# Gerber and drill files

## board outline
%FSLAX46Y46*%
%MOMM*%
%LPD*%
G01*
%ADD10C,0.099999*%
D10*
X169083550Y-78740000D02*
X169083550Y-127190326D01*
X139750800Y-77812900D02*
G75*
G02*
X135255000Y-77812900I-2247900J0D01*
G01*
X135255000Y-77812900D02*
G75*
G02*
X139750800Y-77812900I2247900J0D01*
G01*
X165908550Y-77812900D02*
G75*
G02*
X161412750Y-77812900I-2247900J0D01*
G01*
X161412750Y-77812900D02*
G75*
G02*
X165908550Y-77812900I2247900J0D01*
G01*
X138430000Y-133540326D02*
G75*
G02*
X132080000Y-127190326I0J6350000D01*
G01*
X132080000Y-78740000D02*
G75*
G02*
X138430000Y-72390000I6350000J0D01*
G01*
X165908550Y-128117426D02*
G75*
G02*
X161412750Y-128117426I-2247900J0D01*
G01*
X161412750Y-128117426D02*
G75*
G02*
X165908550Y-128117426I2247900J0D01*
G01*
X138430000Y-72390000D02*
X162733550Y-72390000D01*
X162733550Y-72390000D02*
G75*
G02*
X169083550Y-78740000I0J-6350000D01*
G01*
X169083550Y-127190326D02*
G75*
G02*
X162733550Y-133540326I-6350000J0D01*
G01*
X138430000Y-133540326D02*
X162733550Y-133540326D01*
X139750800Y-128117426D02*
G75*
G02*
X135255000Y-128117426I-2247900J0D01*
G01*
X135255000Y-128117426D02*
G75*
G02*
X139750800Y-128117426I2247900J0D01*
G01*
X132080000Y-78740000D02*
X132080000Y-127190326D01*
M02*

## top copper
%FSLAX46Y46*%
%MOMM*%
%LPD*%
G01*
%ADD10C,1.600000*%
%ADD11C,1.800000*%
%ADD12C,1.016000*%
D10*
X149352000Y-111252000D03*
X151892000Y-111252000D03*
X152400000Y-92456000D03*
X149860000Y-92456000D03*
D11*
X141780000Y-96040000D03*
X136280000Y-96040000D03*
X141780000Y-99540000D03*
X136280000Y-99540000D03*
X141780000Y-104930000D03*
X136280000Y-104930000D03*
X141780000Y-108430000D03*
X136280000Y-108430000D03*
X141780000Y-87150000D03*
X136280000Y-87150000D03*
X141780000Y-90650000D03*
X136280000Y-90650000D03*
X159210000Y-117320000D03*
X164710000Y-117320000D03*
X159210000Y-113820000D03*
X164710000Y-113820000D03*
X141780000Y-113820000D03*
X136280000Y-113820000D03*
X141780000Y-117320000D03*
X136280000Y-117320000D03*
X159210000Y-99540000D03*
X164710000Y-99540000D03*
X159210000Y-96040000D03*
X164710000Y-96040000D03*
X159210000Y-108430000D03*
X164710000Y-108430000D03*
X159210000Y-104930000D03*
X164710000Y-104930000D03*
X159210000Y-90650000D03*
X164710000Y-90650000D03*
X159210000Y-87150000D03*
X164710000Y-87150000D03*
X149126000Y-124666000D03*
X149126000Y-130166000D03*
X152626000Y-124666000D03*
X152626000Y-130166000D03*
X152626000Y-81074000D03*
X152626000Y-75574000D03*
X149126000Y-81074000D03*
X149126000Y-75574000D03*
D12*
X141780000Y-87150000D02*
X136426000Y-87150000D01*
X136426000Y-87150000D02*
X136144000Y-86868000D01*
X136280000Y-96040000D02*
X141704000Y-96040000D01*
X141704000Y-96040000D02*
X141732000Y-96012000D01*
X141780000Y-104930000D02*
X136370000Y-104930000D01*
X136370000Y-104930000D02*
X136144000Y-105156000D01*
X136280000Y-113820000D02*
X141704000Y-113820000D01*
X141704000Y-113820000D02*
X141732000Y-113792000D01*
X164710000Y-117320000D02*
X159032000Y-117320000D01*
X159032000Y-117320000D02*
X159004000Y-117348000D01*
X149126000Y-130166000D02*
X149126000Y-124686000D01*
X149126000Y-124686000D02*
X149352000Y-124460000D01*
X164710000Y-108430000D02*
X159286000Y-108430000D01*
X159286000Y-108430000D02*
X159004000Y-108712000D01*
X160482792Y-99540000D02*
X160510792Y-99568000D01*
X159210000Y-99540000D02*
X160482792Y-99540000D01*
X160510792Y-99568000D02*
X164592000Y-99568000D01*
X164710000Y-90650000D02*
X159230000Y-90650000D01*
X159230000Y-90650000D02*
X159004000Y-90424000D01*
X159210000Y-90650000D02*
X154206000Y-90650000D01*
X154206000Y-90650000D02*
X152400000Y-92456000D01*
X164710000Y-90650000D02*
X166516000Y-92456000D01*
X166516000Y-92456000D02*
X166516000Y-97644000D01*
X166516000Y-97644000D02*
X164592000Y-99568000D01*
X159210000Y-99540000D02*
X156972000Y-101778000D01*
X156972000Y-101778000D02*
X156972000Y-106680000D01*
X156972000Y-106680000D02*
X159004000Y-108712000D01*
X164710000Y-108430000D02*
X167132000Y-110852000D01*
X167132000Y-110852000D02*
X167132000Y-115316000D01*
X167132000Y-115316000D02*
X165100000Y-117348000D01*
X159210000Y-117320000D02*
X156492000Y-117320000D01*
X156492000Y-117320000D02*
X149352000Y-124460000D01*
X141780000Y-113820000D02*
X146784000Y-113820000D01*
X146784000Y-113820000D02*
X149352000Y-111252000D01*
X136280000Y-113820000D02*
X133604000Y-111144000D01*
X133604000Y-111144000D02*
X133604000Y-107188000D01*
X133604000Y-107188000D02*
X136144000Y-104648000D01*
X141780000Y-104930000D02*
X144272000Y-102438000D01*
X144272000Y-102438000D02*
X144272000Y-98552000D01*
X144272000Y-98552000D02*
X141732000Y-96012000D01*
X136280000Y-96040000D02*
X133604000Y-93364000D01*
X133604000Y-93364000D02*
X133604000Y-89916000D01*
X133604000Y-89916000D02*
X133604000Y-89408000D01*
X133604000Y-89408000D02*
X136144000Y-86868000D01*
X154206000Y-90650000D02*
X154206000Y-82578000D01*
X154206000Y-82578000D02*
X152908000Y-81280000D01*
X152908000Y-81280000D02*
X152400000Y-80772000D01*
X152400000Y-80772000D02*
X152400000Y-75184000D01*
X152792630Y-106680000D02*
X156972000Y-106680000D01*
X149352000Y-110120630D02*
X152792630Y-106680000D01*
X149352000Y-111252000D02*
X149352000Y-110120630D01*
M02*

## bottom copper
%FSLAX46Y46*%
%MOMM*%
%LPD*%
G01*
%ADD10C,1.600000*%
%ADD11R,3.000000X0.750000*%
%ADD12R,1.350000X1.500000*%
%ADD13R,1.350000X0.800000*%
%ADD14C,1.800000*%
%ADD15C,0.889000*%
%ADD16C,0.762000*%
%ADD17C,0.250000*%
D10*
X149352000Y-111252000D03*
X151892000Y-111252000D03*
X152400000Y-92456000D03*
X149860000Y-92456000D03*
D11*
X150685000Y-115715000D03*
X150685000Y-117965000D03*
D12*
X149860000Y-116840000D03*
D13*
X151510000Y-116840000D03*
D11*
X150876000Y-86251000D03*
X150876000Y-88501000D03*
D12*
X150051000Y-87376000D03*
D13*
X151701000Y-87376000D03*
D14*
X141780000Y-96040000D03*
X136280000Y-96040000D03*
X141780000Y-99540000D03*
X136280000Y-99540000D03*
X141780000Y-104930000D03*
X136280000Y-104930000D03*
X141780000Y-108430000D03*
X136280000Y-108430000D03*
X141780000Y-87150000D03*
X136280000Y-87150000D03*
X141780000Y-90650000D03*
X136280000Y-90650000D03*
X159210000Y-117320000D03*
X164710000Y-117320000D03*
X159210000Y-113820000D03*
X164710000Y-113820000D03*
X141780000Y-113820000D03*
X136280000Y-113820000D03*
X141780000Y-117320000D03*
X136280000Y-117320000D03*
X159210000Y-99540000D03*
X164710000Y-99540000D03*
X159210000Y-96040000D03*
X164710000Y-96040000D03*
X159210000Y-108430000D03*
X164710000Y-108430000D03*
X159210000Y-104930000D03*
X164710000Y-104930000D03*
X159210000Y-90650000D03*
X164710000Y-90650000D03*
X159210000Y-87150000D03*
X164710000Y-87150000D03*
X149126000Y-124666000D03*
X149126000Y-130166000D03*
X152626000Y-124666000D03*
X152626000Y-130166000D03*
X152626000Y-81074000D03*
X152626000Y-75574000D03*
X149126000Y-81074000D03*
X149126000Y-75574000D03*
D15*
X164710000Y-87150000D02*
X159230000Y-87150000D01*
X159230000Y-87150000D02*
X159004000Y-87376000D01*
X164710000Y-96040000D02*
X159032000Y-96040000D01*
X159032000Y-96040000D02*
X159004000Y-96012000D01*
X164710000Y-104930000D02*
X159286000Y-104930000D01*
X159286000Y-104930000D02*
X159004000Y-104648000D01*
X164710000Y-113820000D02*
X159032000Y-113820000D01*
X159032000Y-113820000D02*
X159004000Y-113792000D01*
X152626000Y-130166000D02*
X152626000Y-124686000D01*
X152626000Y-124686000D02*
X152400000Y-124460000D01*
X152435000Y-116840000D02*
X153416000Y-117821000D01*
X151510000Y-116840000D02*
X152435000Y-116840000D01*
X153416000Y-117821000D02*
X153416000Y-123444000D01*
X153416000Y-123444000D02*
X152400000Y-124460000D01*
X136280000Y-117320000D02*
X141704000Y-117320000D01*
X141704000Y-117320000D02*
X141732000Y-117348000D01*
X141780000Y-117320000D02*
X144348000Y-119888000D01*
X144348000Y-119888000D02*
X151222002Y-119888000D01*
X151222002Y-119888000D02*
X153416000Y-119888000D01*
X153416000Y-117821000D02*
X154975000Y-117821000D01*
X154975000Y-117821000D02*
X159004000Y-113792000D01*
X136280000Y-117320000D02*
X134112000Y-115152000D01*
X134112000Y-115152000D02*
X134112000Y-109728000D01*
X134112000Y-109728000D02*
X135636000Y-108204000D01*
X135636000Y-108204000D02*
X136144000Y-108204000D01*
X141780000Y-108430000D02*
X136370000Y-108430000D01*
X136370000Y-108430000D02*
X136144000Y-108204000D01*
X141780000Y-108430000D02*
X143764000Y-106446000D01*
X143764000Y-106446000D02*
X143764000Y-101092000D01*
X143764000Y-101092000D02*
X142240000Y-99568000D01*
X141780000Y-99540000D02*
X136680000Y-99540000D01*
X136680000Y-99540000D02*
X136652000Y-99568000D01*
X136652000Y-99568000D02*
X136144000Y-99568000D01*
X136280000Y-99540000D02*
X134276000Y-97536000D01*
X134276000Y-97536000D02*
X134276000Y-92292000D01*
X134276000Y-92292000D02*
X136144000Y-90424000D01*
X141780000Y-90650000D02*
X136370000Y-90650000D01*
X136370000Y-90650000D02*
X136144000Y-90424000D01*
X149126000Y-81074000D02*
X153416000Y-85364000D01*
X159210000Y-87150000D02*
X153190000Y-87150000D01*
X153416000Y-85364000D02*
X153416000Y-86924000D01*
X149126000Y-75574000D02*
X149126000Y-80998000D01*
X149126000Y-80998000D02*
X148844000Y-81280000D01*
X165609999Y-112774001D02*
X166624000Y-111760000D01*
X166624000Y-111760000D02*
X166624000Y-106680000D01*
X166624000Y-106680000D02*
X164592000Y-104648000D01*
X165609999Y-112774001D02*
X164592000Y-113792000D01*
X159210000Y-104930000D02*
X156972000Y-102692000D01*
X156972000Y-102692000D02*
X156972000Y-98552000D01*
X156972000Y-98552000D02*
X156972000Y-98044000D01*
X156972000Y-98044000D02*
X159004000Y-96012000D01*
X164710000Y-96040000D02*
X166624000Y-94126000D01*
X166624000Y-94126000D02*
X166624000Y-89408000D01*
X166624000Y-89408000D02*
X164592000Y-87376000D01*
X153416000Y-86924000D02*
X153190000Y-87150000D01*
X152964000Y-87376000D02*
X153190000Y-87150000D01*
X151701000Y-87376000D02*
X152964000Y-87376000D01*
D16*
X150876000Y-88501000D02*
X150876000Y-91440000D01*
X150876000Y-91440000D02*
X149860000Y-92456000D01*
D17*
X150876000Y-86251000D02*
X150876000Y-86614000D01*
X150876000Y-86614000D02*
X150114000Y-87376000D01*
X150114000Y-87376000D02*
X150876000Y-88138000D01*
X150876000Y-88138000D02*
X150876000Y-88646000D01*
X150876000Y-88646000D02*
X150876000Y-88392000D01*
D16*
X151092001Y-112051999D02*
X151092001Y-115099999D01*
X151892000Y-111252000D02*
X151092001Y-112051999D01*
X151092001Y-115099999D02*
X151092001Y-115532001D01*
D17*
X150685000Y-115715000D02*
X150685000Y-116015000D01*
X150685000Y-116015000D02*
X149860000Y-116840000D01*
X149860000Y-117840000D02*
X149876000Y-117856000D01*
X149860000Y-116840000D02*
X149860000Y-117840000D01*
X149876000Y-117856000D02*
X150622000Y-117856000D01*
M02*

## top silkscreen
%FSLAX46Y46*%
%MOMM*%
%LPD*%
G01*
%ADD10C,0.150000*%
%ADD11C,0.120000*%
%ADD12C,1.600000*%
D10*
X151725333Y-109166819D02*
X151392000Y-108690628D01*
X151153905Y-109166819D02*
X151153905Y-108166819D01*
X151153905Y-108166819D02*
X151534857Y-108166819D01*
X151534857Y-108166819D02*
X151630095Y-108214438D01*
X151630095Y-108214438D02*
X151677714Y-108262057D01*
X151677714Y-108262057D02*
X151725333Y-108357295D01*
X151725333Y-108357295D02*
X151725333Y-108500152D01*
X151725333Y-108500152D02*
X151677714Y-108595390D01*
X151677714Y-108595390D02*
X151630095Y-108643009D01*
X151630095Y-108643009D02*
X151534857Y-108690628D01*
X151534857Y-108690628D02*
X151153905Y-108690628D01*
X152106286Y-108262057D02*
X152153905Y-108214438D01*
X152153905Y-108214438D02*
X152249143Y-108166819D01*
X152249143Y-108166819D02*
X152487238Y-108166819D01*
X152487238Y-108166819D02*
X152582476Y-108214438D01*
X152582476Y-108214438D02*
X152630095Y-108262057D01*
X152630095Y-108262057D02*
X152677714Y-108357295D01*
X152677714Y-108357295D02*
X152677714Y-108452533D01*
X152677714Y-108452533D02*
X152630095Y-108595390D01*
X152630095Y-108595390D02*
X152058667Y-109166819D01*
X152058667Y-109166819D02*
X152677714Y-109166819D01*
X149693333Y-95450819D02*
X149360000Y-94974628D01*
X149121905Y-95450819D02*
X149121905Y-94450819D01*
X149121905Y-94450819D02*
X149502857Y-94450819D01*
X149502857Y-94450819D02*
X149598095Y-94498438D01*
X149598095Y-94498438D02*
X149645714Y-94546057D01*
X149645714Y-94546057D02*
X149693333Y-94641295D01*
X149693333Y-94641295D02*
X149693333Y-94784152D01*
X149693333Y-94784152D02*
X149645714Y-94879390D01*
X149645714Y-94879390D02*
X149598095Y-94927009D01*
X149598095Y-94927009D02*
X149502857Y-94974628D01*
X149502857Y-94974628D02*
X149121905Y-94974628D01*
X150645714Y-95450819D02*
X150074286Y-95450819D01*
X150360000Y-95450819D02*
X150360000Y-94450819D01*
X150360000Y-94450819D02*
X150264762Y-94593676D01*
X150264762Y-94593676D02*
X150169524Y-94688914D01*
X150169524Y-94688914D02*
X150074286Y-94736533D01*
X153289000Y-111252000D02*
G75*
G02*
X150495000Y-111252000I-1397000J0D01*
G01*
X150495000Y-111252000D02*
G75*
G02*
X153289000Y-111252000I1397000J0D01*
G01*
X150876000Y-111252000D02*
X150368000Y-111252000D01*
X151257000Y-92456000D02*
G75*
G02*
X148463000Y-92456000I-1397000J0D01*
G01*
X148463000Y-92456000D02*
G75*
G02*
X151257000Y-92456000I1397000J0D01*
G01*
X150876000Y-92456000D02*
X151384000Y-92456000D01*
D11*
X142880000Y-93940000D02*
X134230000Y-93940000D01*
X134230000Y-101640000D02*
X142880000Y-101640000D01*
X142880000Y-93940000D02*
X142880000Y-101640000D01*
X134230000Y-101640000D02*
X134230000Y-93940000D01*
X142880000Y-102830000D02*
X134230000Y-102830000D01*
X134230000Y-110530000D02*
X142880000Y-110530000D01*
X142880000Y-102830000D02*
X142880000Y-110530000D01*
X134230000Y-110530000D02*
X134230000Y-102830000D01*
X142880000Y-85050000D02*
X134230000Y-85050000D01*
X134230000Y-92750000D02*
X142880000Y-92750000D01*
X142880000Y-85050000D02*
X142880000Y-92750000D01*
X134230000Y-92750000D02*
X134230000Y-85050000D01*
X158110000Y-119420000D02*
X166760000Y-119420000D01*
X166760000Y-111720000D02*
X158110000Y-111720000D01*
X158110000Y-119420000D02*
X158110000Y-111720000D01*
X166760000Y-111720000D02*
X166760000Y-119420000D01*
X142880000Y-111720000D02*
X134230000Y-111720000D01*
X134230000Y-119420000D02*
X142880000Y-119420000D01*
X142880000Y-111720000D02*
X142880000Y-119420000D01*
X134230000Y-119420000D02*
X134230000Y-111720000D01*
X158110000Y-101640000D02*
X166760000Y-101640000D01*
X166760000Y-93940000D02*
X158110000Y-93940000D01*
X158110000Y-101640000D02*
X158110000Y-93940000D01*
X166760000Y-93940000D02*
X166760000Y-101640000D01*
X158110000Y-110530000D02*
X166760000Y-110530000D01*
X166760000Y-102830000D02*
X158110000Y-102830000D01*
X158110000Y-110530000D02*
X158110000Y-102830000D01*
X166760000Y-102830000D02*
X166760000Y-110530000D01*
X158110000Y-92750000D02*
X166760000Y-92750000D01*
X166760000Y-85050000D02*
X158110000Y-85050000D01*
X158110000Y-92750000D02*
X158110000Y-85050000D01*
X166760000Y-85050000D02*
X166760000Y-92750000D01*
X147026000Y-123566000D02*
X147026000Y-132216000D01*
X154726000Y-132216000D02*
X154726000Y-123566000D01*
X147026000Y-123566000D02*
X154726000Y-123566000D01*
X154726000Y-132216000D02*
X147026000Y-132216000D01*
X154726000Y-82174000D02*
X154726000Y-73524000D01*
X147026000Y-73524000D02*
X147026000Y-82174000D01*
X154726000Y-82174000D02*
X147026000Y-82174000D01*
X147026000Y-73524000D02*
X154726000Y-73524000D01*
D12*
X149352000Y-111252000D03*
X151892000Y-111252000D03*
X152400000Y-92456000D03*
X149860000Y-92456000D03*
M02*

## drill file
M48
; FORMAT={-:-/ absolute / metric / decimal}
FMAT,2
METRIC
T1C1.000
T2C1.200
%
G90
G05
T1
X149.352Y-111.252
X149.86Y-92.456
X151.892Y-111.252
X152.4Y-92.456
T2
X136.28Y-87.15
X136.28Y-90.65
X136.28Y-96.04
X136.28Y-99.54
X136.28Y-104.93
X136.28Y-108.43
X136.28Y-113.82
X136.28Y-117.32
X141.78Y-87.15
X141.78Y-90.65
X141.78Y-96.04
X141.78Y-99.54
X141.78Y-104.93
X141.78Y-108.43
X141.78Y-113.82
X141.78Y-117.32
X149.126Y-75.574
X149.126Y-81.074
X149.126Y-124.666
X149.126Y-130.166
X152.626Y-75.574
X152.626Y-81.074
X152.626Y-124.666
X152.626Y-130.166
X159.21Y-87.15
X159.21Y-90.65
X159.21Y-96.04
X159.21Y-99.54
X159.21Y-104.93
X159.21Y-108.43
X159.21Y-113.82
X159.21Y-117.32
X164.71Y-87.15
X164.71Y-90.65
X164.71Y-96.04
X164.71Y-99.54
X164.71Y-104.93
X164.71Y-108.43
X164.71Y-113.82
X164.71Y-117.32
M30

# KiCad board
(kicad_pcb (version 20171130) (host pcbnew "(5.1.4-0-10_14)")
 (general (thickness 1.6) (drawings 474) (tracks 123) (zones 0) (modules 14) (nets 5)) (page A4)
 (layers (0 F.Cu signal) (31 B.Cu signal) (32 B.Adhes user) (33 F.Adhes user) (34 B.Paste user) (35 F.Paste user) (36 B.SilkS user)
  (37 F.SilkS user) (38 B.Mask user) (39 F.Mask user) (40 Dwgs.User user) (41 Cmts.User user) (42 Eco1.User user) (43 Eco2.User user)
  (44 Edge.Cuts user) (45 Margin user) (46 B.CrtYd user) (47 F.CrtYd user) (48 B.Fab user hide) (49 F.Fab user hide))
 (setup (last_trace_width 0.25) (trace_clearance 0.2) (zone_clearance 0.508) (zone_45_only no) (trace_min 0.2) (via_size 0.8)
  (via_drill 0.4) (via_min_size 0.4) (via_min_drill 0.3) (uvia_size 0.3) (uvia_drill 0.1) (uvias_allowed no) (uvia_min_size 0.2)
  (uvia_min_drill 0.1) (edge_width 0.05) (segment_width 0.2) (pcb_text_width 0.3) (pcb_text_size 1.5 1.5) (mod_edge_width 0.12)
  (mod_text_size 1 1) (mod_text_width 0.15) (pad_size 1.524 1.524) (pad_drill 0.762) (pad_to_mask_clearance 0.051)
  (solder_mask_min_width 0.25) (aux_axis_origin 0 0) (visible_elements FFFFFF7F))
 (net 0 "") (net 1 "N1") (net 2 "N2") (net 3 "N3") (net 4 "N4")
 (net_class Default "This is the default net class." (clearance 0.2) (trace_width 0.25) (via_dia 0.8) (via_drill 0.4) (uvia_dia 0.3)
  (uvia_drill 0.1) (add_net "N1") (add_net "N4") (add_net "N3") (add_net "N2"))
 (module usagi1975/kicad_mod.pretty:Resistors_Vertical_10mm (layer F.Cu) (at 151.892 111.252 180)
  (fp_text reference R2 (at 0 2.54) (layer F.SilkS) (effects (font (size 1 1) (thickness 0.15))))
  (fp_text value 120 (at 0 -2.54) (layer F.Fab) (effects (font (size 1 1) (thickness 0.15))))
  (fp_circle (center 0 0) (end 1.397 0) (layer F.SilkS) (width 0.15))
  (fp_line (start 1.016 0) (end 1.524 0) (layer F.SilkS) (width 0.15))
  (pad 2 thru_hole circle (at 2.54 0 180) (size 1.6 1.6) (drill 1) (layers *.Cu *.Mask F.SilkS) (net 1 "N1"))
  (pad 1 thru_hole circle (at 0 0 180) (size 1.6 1.6) (drill 1) (layers *.Cu *.Mask F.SilkS) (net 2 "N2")))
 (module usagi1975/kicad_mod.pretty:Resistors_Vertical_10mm (layer F.Cu) (at 149.86 92.456)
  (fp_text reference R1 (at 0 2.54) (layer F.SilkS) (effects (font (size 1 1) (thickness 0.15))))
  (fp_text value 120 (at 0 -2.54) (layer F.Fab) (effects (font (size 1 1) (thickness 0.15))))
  (fp_circle (center 0 0) (end 1.397 0) (layer F.SilkS) (width 0.15))
  (fp_line (start 1.016 0) (end 1.524 0) (layer F.SilkS) (width 0.15))
  (pad 2 thru_hole circle (at 2.54 0) (size 1.6 1.6) (drill 1) (layers *.Cu *.Mask F.SilkS) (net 1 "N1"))
  (pad 1 thru_hole circle (at 0 0) (size 1.6 1.6) (drill 1) (layers *.Cu *.Mask F.SilkS) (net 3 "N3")))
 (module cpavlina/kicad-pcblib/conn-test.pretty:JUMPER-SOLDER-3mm (layer B.Cu) (at 150.685 116.84)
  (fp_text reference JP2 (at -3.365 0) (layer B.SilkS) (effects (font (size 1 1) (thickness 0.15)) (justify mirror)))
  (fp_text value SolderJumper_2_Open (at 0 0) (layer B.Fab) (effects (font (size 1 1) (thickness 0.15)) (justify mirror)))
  (pad 2 smd rect (at 0 -1.125) (size 3 0.75) (layers B.Cu B.Paste B.Mask) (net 2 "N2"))
  (pad 2 smd rect (at 0 1.125) (size 3 0.75) (layers B.Cu B.Paste B.Mask) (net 2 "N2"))
  (pad 2 smd rect (at -0.825 0) (size 1.35 1.5) (layers B.Cu B.Paste B.Mask) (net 2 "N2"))
  (pad 1 smd rect (at 0.825 0) (size 1.35 0.8) (layers B.Cu B.Paste B.Mask) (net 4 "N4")))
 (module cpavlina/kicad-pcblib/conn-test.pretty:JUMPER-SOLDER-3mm (layer B.Cu) (at 150.876 87.376)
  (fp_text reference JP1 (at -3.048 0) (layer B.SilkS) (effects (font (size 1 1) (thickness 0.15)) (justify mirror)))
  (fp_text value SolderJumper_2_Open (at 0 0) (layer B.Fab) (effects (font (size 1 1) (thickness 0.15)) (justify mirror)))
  (pad 2 smd rect (at 0 -1.125) (size 3 0.75) (layers B.Cu B.Paste B.Mask) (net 3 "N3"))
  (pad 2 smd rect (at 0 1.125) (size 3 0.75) (layers B.Cu B.Paste B.Mask) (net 3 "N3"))
  (pad 2 smd rect (at -0.825 0) (size 1.35 1.5) (layers B.Cu B.Paste B.Mask) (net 3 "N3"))
  (pad 1 smd rect (at 0.825 0) (size 1.35 0.8) (layers B.Cu B.Paste B.Mask) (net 4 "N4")))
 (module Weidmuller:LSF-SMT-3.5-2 (layer F.Cu) (at 138.43 97.79 270)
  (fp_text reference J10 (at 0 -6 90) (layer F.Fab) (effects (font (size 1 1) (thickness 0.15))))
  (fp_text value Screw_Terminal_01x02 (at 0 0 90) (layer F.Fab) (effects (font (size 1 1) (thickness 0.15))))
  (fp_line (start -3.85 -4.45) (end -3.85 4.2) (layer F.SilkS) (width 0.12))
  (fp_line (start 3.85 4.2) (end 3.85 -4.45) (layer F.SilkS) (width 0.12))
  (fp_line (start -3.85 -4.45) (end 3.85 -4.45) (layer F.SilkS) (width 0.12))
  (fp_line (start 3.85 4.2) (end -3.85 4.2) (layer F.SilkS) (width 0.12))
  (pad 1 thru_hole circle (at -1.75 -3.35 270) (size 1.8 1.8) (drill 1.2) (layers *.Cu *.Mask) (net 1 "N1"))
  (pad 1 thru_hole circle (at -1.75 2.15 270) (size 1.8 1.8) (drill 1.2) (layers *.Cu *.Mask) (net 1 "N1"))
  (pad 2 thru_hole circle (at 1.75 -3.35 270) (size 1.8 1.8) (drill 1.2) (layers *.Cu *.Mask) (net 4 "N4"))
  (pad 2 thru_hole circle (at 1.75 2.15 270) (size 1.8 1.8) (drill 1.2) (layers *.Cu *.Mask) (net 4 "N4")))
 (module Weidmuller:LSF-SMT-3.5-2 (layer F.Cu) (at 138.43 106.68 270)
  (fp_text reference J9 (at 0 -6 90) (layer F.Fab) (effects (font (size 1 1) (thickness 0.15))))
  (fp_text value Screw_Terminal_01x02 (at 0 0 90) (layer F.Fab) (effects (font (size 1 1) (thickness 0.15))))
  (fp_line (start -3.85 -4.45) (end -3.85 4.2) (layer F.SilkS) (width 0.12))
  (fp_line (start 3.85 4.2) (end 3.85 -4.45) (layer F.SilkS) (width 0.12))
  (fp_line (start -3.85 -4.45) (end 3.85 -4.45) (layer F.SilkS) (width 0.12))
  (fp_line (start 3.85 4.2) (end -3.85 4.2) (layer F.SilkS) (width 0.12))
  (pad 1 thru_hole circle (at -1.75 -3.35 270) (size 1.8 1.8) (drill 1.2) (layers *.Cu *.Mask) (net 1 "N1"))
  (pad 1 thru_hole circle (at -1.75 2.15 270) (size 1.8 1.8) (drill 1.2) (layers *.Cu *.Mask) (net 1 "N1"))
  (pad 2 thru_hole circle (at 1.75 -3.35 270) (size 1.8 1.8) (drill 1.2) (layers *.Cu *.Mask) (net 4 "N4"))
  (pad 2 thru_hole circle (at 1.75 2.15 270) (size 1.8 1.8) (drill 1.2) (layers *.Cu *.Mask) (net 4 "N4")))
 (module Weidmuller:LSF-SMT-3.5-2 (layer F.Cu) (at 138.43 88.9 270)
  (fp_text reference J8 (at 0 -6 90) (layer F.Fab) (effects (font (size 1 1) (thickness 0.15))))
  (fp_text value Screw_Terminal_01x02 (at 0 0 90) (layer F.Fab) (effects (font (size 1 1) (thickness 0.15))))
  (fp_line (start -3.85 -4.45) (end -3.85 4.2) (layer F.SilkS) (width 0.12))
  (fp_line (start 3.85 4.2) (end 3.85 -4.45) (layer F.SilkS) (width 0.12))
  (fp_line (start -3.85 -4.45) (end 3.85 -4.45) (layer F.SilkS) (width 0.12))
  (fp_line (start 3.85 4.2) (end -3.85 4.2) (layer F.SilkS) (width 0.12))
  (pad 1 thru_hole circle (at -1.75 -3.35 270) (size 1.8 1.8) (drill 1.2) (layers *.Cu *.Mask) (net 1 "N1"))
  (pad 1 thru_hole circle (at -1.75 2.15 270) (size 1.8 1.8) (drill 1.2) (layers *.Cu *.Mask) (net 1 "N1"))
  (pad 2 thru_hole circle (at 1.75 -3.35 270) (size 1.8 1.8) (drill 1.2) (layers *.Cu *.Mask) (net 4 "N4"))
  (pad 2 thru_hole circle (at 1.75 2.15 270) (size 1.8 1.8) (drill 1.2) (layers *.Cu *.Mask) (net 4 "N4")))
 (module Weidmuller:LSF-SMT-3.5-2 (layer F.Cu) (at 162.56 115.57 90)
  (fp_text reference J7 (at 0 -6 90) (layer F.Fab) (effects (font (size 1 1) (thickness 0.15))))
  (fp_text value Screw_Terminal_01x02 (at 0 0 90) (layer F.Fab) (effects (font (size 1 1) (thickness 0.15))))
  (fp_line (start -3.85 -4.45) (end -3.85 4.2) (layer F.SilkS) (width 0.12))
  (fp_line (start 3.85 4.2) (end 3.85 -4.45) (layer F.SilkS) (width 0.12))
  (fp_line (start -3.85 -4.45) (end 3.85 -4.45) (layer F.SilkS) (width 0.12))
  (fp_line (start 3.85 4.2) (end -3.85 4.2) (layer F.SilkS) (width 0.12))
  (pad 1 thru_hole circle (at -1.75 -3.35 90) (size 1.8 1.8) (drill 1.2) (layers *.Cu *.Mask) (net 1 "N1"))
  (pad 1 thru_hole circle (at -1.75 2.15 90) (size 1.8 1.8) (drill 1.2) (layers *.Cu *.Mask) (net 1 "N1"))
  (pad 2 thru_hole circle (at 1.75 -3.35 90) (size 1.8 1.8) (drill 1.2) (layers *.Cu *.Mask) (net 4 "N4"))
  (pad 2 thru_hole circle (at 1.75 2.15 90) (size 1.8 1.8) (drill 1.2) (layers *.Cu *.Mask) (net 4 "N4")))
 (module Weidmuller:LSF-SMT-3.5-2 (layer F.Cu) (at 138.43 115.57 270)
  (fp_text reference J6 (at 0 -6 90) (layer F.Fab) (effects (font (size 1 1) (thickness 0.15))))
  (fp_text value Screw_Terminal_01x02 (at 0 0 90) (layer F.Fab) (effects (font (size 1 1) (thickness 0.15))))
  (fp_line (start -3.85 -4.45) (end -3.85 4.2) (layer F.SilkS) (width 0.12))
  (fp_line (start 3.85 4.2) (end 3.85 -4.45) (layer F.SilkS) (width 0.12))
  (fp_line (start -3.85 -4.45) (end 3.85 -4.45) (layer F.SilkS) (width 0.12))
  (fp_line (start 3.85 4.2) (end -3.85 4.2) (layer F.SilkS) (width 0.12))
  (pad 1 thru_hole circle (at -1.75 -3.35 270) (size 1.8 1.8) (drill 1.2) (layers *.Cu *.Mask) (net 1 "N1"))
  (pad 1 thru_hole circle (at -1.75 2.15 270) (size 1.8 1.8) (drill 1.2) (layers *.Cu *.Mask) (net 1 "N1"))
  (pad 2 thru_hole circle (at 1.75 -3.35 270) (size 1.8 1.8) (drill 1.2) (layers *.Cu *.Mask) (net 4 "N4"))
  (pad 2 thru_hole circle (at 1.75 2.15 270) (size 1.8 1.8) (drill 1.2) (layers *.Cu *.Mask) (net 4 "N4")))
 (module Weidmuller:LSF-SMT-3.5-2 (layer F.Cu) (at 162.56 97.79 90)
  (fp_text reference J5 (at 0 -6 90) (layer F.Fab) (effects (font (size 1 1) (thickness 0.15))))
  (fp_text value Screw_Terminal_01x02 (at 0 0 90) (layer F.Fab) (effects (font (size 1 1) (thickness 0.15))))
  (fp_line (start -3.85 -4.45) (end -3.85 4.2) (layer F.SilkS) (width 0.12))
  (fp_line (start 3.85 4.2) (end 3.85 -4.45) (layer F.SilkS) (width 0.12))
  (fp_line (start -3.85 -4.45) (end 3.85 -4.45) (layer F.SilkS) (width 0.12))
  (fp_line (start 3.85 4.2) (end -3.85 4.2) (layer F.SilkS) (width 0.12))
  (pad 1 thru_hole circle (at -1.75 -3.35 90) (size 1.8 1.8) (drill 1.2) (layers *.Cu *.Mask) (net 1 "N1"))
  (pad 1 thru_hole circle (at -1.75 2.15 90) (size 1.8 1.8) (drill 1.2) (layers *.Cu *.Mask) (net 1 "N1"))
  (pad 2 thru_hole circle (at 1.75 -3.35 90) (size 1.8 1.8) (drill 1.2) (layers *.Cu *.Mask) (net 4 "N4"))
  (pad 2 thru_hole circle (at 1.75 2.15 90) (size 1.8 1.8) (drill 1.2) (layers *.Cu *.Mask) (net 4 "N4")))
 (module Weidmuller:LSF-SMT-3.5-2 (layer F.Cu) (at 162.56 106.68 90)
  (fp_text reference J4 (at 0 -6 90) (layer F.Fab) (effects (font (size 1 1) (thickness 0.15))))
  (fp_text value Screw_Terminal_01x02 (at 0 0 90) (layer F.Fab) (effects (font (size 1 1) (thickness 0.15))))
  (fp_line (start -3.85 -4.45) (end -3.85 4.2) (layer F.SilkS) (width 0.12))
  (fp_line (start 3.85 4.2) (end 3.85 -4.45) (layer F.SilkS) (width 0.12))
  (fp_line (start -3.85 -4.45) (end 3.85 -4.45) (layer F.SilkS) (width 0.12))
  (fp_line (start 3.85 4.2) (end -3.85 4.2) (layer F.SilkS) (width 0.12))
  (pad 1 thru_hole circle (at -1.75 -3.35 90) (size 1.8 1.8) (drill 1.2) (layers *.Cu *.Mask) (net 1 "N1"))
  (pad 1 thru_hole circle (at -1.75 2.15 90) (size 1.8 1.8) (drill 1.2) (layers *.Cu *.Mask) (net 1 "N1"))
  (pad 2 thru_hole circle (at 1.75 -3.35 90) (size 1.8 1.8) (drill 1.2) (layers *.Cu *.Mask) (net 4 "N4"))
  (pad 2 thru_hole circle (at 1.75 2.15 90) (size 1.8 1.8) (drill 1.2) (layers *.Cu *.Mask) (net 4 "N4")))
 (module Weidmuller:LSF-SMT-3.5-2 (layer F.Cu) (at 162.56 88.9 90)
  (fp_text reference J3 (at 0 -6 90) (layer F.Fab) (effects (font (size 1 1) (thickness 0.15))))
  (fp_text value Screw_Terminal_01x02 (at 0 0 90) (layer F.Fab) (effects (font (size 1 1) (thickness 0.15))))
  (fp_line (start -3.85 -4.45) (end -3.85 4.2) (layer F.SilkS) (width 0.12))
  (fp_line (start 3.85 4.2) (end 3.85 -4.45) (layer F.SilkS) (width 0.12))
  (fp_line (start -3.85 -4.45) (end 3.85 -4.45) (layer F.SilkS) (width 0.12))
  (fp_line (start 3.85 4.2) (end -3.85 4.2) (layer F.SilkS) (width 0.12))
  (pad 1 thru_hole circle (at -1.75 -3.35 90) (size 1.8 1.8) (drill 1.2) (layers *.Cu *.Mask) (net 1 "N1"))
  (pad 1 thru_hole circle (at -1.75 2.15 90) (size 1.8 1.8) (drill 1.2) (layers *.Cu *.Mask) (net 1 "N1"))
  (pad 2 thru_hole circle (at 1.75 -3.35 90) (size 1.8 1.8) (drill 1.2) (layers *.Cu *.Mask) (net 4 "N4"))
  (pad 2 thru_hole circle (at 1.75 2.15 90) (size 1.8 1.8) (drill 1.2) (layers *.Cu *.Mask) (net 4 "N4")))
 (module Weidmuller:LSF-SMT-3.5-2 (layer F.Cu) (at 150.876 128.016)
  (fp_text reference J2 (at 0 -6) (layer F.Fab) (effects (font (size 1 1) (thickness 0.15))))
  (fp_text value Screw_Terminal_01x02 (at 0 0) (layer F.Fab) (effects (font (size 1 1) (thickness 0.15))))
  (fp_line (start -3.85 -4.45) (end -3.85 4.2) (layer F.SilkS) (width 0.12))
  (fp_line (start 3.85 4.2) (end 3.85 -4.45) (layer F.SilkS) (width 0.12))
  (fp_line (start -3.85 -4.45) (end 3.85 -4.45) (layer F.SilkS) (width 0.12))
  (fp_line (start 3.85 4.2) (end -3.85 4.2) (layer F.SilkS) (width 0.12))
  (pad 1 thru_hole circle (at -1.75 -3.35) (size 1.8 1.8) (drill 1.2) (layers *.Cu *.Mask) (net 1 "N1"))
  (pad 1 thru_hole circle (at -1.75 2.15) (size 1.8 1.8) (drill 1.2) (layers *.Cu *.Mask) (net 1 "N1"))
  (pad 2 thru_hole circle (at 1.75 -3.35) (size 1.8 1.8) (drill 1.2) (layers *.Cu *.Mask) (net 4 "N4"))
  (pad 2 thru_hole circle (at 1.75 2.15) (size 1.8 1.8) (drill 1.2) (layers *.Cu *.Mask) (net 4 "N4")))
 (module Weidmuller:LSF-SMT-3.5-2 (layer F.Cu) (at 150.876 77.724 180)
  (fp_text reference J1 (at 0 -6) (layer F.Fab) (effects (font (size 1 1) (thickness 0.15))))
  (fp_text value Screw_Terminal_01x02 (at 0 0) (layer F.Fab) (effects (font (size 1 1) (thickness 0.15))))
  (fp_line (start -3.85 -4.45) (end -3.85 4.2) (layer F.SilkS) (width 0.12))
  (fp_line (start 3.85 4.2) (end 3.85 -4.45) (layer F.SilkS) (width 0.12))
  (fp_line (start -3.85 -4.45) (end 3.85 -4.45) (layer F.SilkS) (width 0.12))
  (fp_line (start 3.85 4.2) (end -3.85 4.2) (layer F.SilkS) (width 0.12))
  (pad 1 thru_hole circle (at -1.75 -3.35 180) (size 1.8 1.8) (drill 1.2) (layers *.Cu *.Mask) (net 1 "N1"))
  (pad 1 thru_hole circle (at -1.75 2.15 180) (size 1.8 1.8) (drill 1.2) (layers *.Cu *.Mask) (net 1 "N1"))
  (pad 2 thru_hole circle (at 1.75 -3.35 180) (size 1.8 1.8) (drill 1.2) (layers *.Cu *.Mask) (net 4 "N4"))
  (pad 2 thru_hole circle (at 1.75 2.15 180) (size 1.8 1.8) (drill 1.2) (layers *.Cu *.Mask) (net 4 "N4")))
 (gr_line (start 169.08355 78.74) (end 169.08355 127.190326) (layer Edge.Cuts) (width 0.099999))
 (gr_circle (center 137.5029 77.8129) (end 139.7508 77.8129) (layer Edge.Cuts) (width 0.099999))
 (gr_circle (center 163.66065 77.8129) (end 165.90855 77.8129) (layer Edge.Cuts) (width 0.099999))
 (gr_arc (start 138.43 127.190326) (end 132.08 127.190326) (angle -90) (layer Edge.Cuts) (width 0.099999))
 (gr_arc (start 138.43 78.74) (end 138.43 72.39) (angle -90) (layer Edge.Cuts) (width 0.099999))
 (gr_circle (center 163.66065 128.117426) (end 165.90855 128.117426) (layer Edge.Cuts) (width 0.099999))
 (gr_line (start 138.43 72.39) (end 162.73355 72.39) (layer Edge.Cuts) (width 0.099999))
 (gr_arc (start 162.73355 78.74) (end 169.08355 78.74) (angle -90) (layer Edge.Cuts) (width 0.099999))
 (gr_arc (start 162.73355 127.190326) (end 162.73355 133.540326) (angle -90) (layer Edge.Cuts) (width 0.099999))
 (gr_line (start 138.43 133.540326) (end 162.73355 133.540326) (layer Edge.Cuts) (width 0.099999))
 (gr_circle (center 137.5029 128.117426) (end 139.7508 128.117426) (layer Edge.Cuts) (width 0.099999))
 (gr_line (start 132.08 78.74) (end 132.08 127.190326) (layer Edge.Cuts) (width 0.099999))
 (segment (start 141.78 87.15) (end 136.426 87.15) (width 1.016) (layer F.Cu) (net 1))
 (segment (start 136.426 87.15) (end 136.144 86.868) (width 1.016) (layer F.Cu) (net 1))
 (segment (start 136.28 96.04) (end 141.704 96.04) (width 1.016) (layer F.Cu) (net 1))
 (segment (start 141.704 96.04) (end 141.732 96.012) (width 1.016) (layer F.Cu) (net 1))
 (segment (start 141.78 104.93) (end 136.37 104.93) (width 1.016) (layer F.Cu) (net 1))
 (segment (start 136.37 104.93) (end 136.144 105.156) (width 1.016) (layer F.Cu) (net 1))
 (segment (start 136.28 113.82) (end 141.704 113.82) (width 1.016) (layer F.Cu) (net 1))
 (segment (start 141.704 113.82) (end 141.732 113.792) (width 1.016) (layer F.Cu) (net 1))
 (segment (start 164.71 117.32) (end 159.032 117.32) (width 1.016) (layer F.Cu) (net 1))
 (segment (start 159.032 117.32) (end 159.004 117.348) (width 1.016) (layer F.Cu) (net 1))
 (segment (start 149.126 130.166) (end 149.126 124.686) (width 1.016) (layer F.Cu) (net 1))
 (segment (start 149.126 124.686) (end 149.352 124.46) (width 1.016) (layer F.Cu) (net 1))
 (segment (start 164.71 108.43) (end 159.286 108.43) (width 1.016) (layer F.Cu) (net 1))
 (segment (start 159.286 108.43) (end 159.004 108.712) (width 1.016) (layer F.Cu) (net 1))
 (segment (start 160.482792 99.54) (end 160.510792 99.568) (width 1.016) (layer F.Cu) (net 1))
 (segment (start 159.21 99.54) (end 160.482792 99.54) (width 1.016) (layer F.Cu) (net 1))
 (segment (start 160.510792 99.568) (end 164.592 99.568) (width 1.016) (layer F.Cu) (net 1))
 (segment (start 164.71 90.65) (end 159.23 90.65) (width 1.016) (layer F.Cu) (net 1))
 (segment (start 159.23 90.65) (end 159.004 90.424) (width 1.016) (layer F.Cu) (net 1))
 (segment (start 159.21 90.65) (end 154.206 90.65) (width 1.016) (layer F.Cu) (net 1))
 (segment (start 154.206 90.65) (end 152.4 92.456) (width 1.016) (layer F.Cu) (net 1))
 (segment (start 164.71 90.65) (end 166.516 92.456) (width 1.016) (layer F.Cu) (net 1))
 (segment (start 166.516 92.456) (end 166.516 97.644) (width 1.016) (layer F.Cu) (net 1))
 (segment (start 166.516 97.644) (end 164.592 99.568) (width 1.016) (layer F.Cu) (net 1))
 (segment (start 159.21 99.54) (end 156.972 101.778) (width 1.016) (layer F.Cu) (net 1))
 (segment (start 156.972 101.778) (end 156.972 106.68) (width 1.016) (layer F.Cu) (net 1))
 (segment (start 156.972 106.68) (end 159.004 108.712) (width 1.016) (layer F.Cu) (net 1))
 (segment (start 164.71 108.43) (end 167.132 110.852) (width 1.016) (layer F.Cu) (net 1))
 (segment (start 167.132 110.852) (end 167.132 115.316) (width 1.016) (layer F.Cu) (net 1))
 (segment (start 167.132 115.316) (end 165.1 117.348) (width 1.016) (layer F.Cu) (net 1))
 (segment (start 159.21 117.32) (end 156.492 117.32) (width 1.016) (layer F.Cu) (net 1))
 (segment (start 156.492 117.32) (end 149.352 124.46) (width 1.016) (layer F.Cu) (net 1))
 (segment (start 141.78 113.82) (end 146.784 113.82) (width 1.016) (layer F.Cu) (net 1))
 (segment (start 146.784 113.82) (end 149.352 111.252) (width 1.016) (layer F.Cu) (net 1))
 (segment (start 136.28 113.82) (end 133.604 111.144) (width 1.016) (layer F.Cu) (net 1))
 (segment (start 133.604 111.144) (end 133.604 107.188) (width 1.016) (layer F.Cu) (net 1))
 (segment (start 133.604 107.188) (end 136.144 104.648) (width 1.016) (layer F.Cu) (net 1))
 (segment (start 141.78 104.93) (end 144.272 102.438) (width 1.016) (layer F.Cu) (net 1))
 (segment (start 144.272 102.438) (end 144.272 98.552) (width 1.016) (layer F.Cu) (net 1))
 (segment (start 144.272 98.552) (end 141.732 96.012) (width 1.016) (layer F.Cu) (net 1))
 (segment (start 136.28 96.04) (end 133.604 93.364) (width 1.016) (layer F.Cu) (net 1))
 (segment (start 133.604 93.364) (end 133.604 89.916) (width 1.016) (layer F.Cu) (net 1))
 (segment (start 133.604 89.916) (end 133.604 89.408) (width 1.016) (layer F.Cu) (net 1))
 (segment (start 133.604 89.408) (end 136.144 86.868) (width 1.016) (layer F.Cu) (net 1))
 (segment (start 154.206 90.65) (end 154.206 82.578) (width 1.016) (layer F.Cu) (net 1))
 (segment (start 154.206 82.578) (end 152.908 81.28) (width 1.016) (layer F.Cu) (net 1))
 (segment (start 152.908 81.28) (end 152.4 80.772) (width 1.016) (layer F.Cu) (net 1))
 (segment (start 152.4 80.772) (end 152.4 75.184) (width 1.016) (layer F.Cu) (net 1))
 (segment (start 152.79263 106.68) (end 156.972 106.68) (width 1.016) (layer F.Cu) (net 1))
 (segment (start 149.352 110.12063) (end 152.79263 106.68) (width 1.016) (layer F.Cu) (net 1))
 (segment (start 149.352 111.252) (end 149.352 110.12063) (width 1.016) (layer F.Cu) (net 1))
 (segment (start 164.71 87.15) (end 159.23 87.15) (width 0.889) (layer B.Cu) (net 4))
 (segment (start 159.23 87.15) (end 159.004 87.376) (width 0.889) (layer B.Cu) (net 4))
 (segment (start 164.71 96.04) (end 159.032 96.04) (width 0.889) (layer B.Cu) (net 4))
 (segment (start 159.032 96.04) (end 159.004 96.012) (width 0.889) (layer B.Cu) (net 4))
 (segment (start 164.71 104.93) (end 159.286 104.93) (width 0.889) (layer B.Cu) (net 4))
 (segment (start 159.286 104.93) (end 159.004 104.648) (width 0.889) (layer B.Cu) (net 4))
 (segment (start 164.71 113.82) (end 159.032 113.82) (width 0.889) (layer B.Cu) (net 4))
 (segment (start 159.032 113.82) (end 159.004 113.792) (width 0.889) (layer B.Cu) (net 4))
 (segment (start 152.626 130.166) (end 152.626 124.686) (width 0.889) (layer B.Cu) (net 4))
 (segment (start 152.626 124.686) (end 152.4 124.46) (width 0.889) (layer B.Cu) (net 4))
 (segment (start 152.435 116.84) (end 153.416 117.821) (width 0.889) (layer B.Cu) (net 4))
 (segment (start 151.51 116.84) (end 152.435 116.84) (width 0.889) (layer B.Cu) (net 4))
 (segment (start 153.416 117.821) (end 153.416 123.444) (width 0.889) (layer B.Cu) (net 4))
 (segment (start 153.416 123.444) (end 152.4 124.46) (width 0.889) (layer B.Cu) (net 4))
 (segment (start 136.28 117.32) (end 141.704 117.32) (width 0.889) (layer B.Cu) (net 4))
 (segment (start 141.704 117.32) (end 141.732 117.348) (width 0.889) (layer B.Cu) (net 4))
 (segment (start 141.78 117.32) (end 144.348 119.888) (width 0.889) (layer B.Cu) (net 4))
 (segment (start 144.348 119.888) (end 151.222002 119.888) (width 0.889) (layer B.Cu) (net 4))
 (segment (start 151.222002 119.888) (end 153.416 119.888) (width 0.889) (layer B.Cu) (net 4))
 (segment (start 153.416 117.821) (end 154.975 117.821) (width 0.889) (layer B.Cu) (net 4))
 (segment (start 154.975 117.821) (end 159.004 113.792) (width 0.889) (layer B.Cu) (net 4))
 (segment (start 136.28 117.32) (end 134.112 115.152) (width 0.889) (layer B.Cu) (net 4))
 (segment (start 134.112 115.152) (end 134.112 109.728) (width 0.889) (layer B.Cu) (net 4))
 (segment (start 134.112 109.728) (end 135.636 108.204) (width 0.889) (layer B.Cu) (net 4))
 (segment (start 135.636 108.204) (end 136.144 108.204) (width 0.889) (layer B.Cu) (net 4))
 (segment (start 141.78 108.43) (end 136.37 108.43) (width 0.889) (layer B.Cu) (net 4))
 (segment (start 136.37 108.43) (end 136.144 108.204) (width 0.889) (layer B.Cu) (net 4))
 (segment (start 141.78 108.43) (end 143.764 106.446) (width 0.889) (layer B.Cu) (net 4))
 (segment (start 143.764 106.446) (end 143.764 101.092) (width 0.889) (layer B.Cu) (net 4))
 (segment (start 143.764 101.092) (end 142.24 99.568) (width 0.889) (layer B.Cu) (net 4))
 (segment (start 141.78 99.54) (end 136.68 99.54) (width 0.889) (layer B.Cu) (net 4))
 (segment (start 136.68 99.54) (end 136.652 99.568) (width 0.889) (layer B.Cu) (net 4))
 (segment (start 136.652 99.568) (end 136.144 99.568) (width 0.889) (layer B.Cu) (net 4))
 (segment (start 136.28 99.54) (end 134.276 97.536) (width 0.889) (layer B.Cu) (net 4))
 (segment (start 134.276 97.536) (end 134.276 92.292) (width 0.889) (layer B.Cu) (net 4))
 (segment (start 134.276 92.292) (end 136.144 90.424) (width 0.889) (layer B.Cu) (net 4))
 (segment (start 141.78 90.65) (end 136.37 90.65) (width 0.889) (layer B.Cu) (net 4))
 (segment (start 136.37 90.65) (end 136.144 90.424) (width 0.889) (layer B.Cu) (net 4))
 (segment (start 149.126 81.074) (end 153.416 85.364) (width 0.889) (layer B.Cu) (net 4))
 (segment (start 159.21 87.15) (end 153.19 87.15) (width 0.889) (layer B.Cu) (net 4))
 (segment (start 153.416 85.364) (end 153.416 86.924) (width 0.889) (layer B.Cu) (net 4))
 (segment (start 149.126 75.574) (end 149.126 80.998) (width 0.889) (layer B.Cu) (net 4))
 (segment (start 149.126 80.998) (end 148.844 81.28) (width 0.889) (layer B.Cu) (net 4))
 (segment (start 165.609999 112.774001) (end 166.624 111.76) (width 0.889) (layer B.Cu) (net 4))
 (segment (start 166.624 111.76) (end 166.624 106.68) (width 0.889) (layer B.Cu) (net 4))
 (segment (start 166.624 106.68) (end 164.592 104.648) (width 0.889) (layer B.Cu) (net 4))
 (segment (start 165.609999 112.774001) (end 164.592 113.792) (width 0.889) (layer B.Cu) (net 4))
 (segment (start 159.21 104.93) (end 156.972 102.692) (width 0.889) (layer B.Cu) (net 4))
 (segment (start 156.972 102.692) (end 156.972 98.552) (width 0.889) (layer B.Cu) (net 4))
 (segment (start 156.972 98.552) (end 156.972 98.044) (width 0.889) (layer B.Cu) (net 4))
 (segment (start 156.972 98.044) (end 159.004 96.012) (width 0.889) (layer B.Cu) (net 4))
 (segment (start 164.71 96.04) (end 166.624 94.126) (width 0.889) (layer B.Cu) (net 4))
 (segment (start 166.624 94.126) (end 166.624 89.408) (width 0.889) (layer B.Cu) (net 4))
 (segment (start 166.624 89.408) (end 164.592 87.376) (width 0.889) (layer B.Cu) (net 4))
 (segment (start 153.416 86.924) (end 153.19 87.15) (width 0.889) (layer B.Cu) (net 4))
 (segment (start 152.964 87.376) (end 153.19 87.15) (width 0.889) (layer B.Cu) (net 4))
 (segment (start 151.701 87.376) (end 152.964 87.376) (width 0.889) (layer B.Cu) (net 4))
 (segment (start 150.876 88.501) (end 150.876 91.44) (width 0.762) (layer B.Cu) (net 3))
 (segment (start 150.876 91.44) (end 149.86 92.456) (width 0.762) (layer B.Cu) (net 3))
 (segment (start 150.876 86.251) (end 150.876 86.614) (width 0.25) (layer B.Cu) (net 3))
 (segment (start 150.876 86.614) (end 150.114 87.376) (width 0.25) (layer B.Cu) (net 3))
 (segment (start 150.114 87.376) (end 150.876 88.138) (width 0.25) (layer B.Cu) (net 3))
 (segment (start 150.876 88.138) (end 150.876 88.646) (width 0.25) (layer B.Cu) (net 3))
 (segment (start 150.876 88.646) (end 150.876 88.392) (width 0.25) (layer B.Cu) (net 3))
 (segment (start 151.092001 112.051999) (end 151.092001 115.099999) (width 0.762) (layer B.Cu) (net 2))
 (segment (start 151.892 111.252) (end 151.092001 112.051999) (width 0.762) (layer B.Cu) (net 2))
 (segment (start 151.092001 115.099999) (end 151.092001 115.532001) (width 0.762) (layer B.Cu) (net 2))
 (segment (start 150.685 115.715) (end 150.685 116.015) (width 0.25) (layer B.Cu) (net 2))
 (segment (start 150.685 116.015) (end 149.86 116.84) (width 0.25) (layer B.Cu) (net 2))
 (segment (start 149.86 117.84) (end 149.876 117.856) (width 0.25) (layer B.Cu) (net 2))
 (segment (start 149.86 116.84) (end 149.86 117.84) (width 0.25) (layer B.Cu) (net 2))
 (segment (start 149.876 117.856) (end 150.622 117.856) (width 0.25) (layer B.Cu) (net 2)))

